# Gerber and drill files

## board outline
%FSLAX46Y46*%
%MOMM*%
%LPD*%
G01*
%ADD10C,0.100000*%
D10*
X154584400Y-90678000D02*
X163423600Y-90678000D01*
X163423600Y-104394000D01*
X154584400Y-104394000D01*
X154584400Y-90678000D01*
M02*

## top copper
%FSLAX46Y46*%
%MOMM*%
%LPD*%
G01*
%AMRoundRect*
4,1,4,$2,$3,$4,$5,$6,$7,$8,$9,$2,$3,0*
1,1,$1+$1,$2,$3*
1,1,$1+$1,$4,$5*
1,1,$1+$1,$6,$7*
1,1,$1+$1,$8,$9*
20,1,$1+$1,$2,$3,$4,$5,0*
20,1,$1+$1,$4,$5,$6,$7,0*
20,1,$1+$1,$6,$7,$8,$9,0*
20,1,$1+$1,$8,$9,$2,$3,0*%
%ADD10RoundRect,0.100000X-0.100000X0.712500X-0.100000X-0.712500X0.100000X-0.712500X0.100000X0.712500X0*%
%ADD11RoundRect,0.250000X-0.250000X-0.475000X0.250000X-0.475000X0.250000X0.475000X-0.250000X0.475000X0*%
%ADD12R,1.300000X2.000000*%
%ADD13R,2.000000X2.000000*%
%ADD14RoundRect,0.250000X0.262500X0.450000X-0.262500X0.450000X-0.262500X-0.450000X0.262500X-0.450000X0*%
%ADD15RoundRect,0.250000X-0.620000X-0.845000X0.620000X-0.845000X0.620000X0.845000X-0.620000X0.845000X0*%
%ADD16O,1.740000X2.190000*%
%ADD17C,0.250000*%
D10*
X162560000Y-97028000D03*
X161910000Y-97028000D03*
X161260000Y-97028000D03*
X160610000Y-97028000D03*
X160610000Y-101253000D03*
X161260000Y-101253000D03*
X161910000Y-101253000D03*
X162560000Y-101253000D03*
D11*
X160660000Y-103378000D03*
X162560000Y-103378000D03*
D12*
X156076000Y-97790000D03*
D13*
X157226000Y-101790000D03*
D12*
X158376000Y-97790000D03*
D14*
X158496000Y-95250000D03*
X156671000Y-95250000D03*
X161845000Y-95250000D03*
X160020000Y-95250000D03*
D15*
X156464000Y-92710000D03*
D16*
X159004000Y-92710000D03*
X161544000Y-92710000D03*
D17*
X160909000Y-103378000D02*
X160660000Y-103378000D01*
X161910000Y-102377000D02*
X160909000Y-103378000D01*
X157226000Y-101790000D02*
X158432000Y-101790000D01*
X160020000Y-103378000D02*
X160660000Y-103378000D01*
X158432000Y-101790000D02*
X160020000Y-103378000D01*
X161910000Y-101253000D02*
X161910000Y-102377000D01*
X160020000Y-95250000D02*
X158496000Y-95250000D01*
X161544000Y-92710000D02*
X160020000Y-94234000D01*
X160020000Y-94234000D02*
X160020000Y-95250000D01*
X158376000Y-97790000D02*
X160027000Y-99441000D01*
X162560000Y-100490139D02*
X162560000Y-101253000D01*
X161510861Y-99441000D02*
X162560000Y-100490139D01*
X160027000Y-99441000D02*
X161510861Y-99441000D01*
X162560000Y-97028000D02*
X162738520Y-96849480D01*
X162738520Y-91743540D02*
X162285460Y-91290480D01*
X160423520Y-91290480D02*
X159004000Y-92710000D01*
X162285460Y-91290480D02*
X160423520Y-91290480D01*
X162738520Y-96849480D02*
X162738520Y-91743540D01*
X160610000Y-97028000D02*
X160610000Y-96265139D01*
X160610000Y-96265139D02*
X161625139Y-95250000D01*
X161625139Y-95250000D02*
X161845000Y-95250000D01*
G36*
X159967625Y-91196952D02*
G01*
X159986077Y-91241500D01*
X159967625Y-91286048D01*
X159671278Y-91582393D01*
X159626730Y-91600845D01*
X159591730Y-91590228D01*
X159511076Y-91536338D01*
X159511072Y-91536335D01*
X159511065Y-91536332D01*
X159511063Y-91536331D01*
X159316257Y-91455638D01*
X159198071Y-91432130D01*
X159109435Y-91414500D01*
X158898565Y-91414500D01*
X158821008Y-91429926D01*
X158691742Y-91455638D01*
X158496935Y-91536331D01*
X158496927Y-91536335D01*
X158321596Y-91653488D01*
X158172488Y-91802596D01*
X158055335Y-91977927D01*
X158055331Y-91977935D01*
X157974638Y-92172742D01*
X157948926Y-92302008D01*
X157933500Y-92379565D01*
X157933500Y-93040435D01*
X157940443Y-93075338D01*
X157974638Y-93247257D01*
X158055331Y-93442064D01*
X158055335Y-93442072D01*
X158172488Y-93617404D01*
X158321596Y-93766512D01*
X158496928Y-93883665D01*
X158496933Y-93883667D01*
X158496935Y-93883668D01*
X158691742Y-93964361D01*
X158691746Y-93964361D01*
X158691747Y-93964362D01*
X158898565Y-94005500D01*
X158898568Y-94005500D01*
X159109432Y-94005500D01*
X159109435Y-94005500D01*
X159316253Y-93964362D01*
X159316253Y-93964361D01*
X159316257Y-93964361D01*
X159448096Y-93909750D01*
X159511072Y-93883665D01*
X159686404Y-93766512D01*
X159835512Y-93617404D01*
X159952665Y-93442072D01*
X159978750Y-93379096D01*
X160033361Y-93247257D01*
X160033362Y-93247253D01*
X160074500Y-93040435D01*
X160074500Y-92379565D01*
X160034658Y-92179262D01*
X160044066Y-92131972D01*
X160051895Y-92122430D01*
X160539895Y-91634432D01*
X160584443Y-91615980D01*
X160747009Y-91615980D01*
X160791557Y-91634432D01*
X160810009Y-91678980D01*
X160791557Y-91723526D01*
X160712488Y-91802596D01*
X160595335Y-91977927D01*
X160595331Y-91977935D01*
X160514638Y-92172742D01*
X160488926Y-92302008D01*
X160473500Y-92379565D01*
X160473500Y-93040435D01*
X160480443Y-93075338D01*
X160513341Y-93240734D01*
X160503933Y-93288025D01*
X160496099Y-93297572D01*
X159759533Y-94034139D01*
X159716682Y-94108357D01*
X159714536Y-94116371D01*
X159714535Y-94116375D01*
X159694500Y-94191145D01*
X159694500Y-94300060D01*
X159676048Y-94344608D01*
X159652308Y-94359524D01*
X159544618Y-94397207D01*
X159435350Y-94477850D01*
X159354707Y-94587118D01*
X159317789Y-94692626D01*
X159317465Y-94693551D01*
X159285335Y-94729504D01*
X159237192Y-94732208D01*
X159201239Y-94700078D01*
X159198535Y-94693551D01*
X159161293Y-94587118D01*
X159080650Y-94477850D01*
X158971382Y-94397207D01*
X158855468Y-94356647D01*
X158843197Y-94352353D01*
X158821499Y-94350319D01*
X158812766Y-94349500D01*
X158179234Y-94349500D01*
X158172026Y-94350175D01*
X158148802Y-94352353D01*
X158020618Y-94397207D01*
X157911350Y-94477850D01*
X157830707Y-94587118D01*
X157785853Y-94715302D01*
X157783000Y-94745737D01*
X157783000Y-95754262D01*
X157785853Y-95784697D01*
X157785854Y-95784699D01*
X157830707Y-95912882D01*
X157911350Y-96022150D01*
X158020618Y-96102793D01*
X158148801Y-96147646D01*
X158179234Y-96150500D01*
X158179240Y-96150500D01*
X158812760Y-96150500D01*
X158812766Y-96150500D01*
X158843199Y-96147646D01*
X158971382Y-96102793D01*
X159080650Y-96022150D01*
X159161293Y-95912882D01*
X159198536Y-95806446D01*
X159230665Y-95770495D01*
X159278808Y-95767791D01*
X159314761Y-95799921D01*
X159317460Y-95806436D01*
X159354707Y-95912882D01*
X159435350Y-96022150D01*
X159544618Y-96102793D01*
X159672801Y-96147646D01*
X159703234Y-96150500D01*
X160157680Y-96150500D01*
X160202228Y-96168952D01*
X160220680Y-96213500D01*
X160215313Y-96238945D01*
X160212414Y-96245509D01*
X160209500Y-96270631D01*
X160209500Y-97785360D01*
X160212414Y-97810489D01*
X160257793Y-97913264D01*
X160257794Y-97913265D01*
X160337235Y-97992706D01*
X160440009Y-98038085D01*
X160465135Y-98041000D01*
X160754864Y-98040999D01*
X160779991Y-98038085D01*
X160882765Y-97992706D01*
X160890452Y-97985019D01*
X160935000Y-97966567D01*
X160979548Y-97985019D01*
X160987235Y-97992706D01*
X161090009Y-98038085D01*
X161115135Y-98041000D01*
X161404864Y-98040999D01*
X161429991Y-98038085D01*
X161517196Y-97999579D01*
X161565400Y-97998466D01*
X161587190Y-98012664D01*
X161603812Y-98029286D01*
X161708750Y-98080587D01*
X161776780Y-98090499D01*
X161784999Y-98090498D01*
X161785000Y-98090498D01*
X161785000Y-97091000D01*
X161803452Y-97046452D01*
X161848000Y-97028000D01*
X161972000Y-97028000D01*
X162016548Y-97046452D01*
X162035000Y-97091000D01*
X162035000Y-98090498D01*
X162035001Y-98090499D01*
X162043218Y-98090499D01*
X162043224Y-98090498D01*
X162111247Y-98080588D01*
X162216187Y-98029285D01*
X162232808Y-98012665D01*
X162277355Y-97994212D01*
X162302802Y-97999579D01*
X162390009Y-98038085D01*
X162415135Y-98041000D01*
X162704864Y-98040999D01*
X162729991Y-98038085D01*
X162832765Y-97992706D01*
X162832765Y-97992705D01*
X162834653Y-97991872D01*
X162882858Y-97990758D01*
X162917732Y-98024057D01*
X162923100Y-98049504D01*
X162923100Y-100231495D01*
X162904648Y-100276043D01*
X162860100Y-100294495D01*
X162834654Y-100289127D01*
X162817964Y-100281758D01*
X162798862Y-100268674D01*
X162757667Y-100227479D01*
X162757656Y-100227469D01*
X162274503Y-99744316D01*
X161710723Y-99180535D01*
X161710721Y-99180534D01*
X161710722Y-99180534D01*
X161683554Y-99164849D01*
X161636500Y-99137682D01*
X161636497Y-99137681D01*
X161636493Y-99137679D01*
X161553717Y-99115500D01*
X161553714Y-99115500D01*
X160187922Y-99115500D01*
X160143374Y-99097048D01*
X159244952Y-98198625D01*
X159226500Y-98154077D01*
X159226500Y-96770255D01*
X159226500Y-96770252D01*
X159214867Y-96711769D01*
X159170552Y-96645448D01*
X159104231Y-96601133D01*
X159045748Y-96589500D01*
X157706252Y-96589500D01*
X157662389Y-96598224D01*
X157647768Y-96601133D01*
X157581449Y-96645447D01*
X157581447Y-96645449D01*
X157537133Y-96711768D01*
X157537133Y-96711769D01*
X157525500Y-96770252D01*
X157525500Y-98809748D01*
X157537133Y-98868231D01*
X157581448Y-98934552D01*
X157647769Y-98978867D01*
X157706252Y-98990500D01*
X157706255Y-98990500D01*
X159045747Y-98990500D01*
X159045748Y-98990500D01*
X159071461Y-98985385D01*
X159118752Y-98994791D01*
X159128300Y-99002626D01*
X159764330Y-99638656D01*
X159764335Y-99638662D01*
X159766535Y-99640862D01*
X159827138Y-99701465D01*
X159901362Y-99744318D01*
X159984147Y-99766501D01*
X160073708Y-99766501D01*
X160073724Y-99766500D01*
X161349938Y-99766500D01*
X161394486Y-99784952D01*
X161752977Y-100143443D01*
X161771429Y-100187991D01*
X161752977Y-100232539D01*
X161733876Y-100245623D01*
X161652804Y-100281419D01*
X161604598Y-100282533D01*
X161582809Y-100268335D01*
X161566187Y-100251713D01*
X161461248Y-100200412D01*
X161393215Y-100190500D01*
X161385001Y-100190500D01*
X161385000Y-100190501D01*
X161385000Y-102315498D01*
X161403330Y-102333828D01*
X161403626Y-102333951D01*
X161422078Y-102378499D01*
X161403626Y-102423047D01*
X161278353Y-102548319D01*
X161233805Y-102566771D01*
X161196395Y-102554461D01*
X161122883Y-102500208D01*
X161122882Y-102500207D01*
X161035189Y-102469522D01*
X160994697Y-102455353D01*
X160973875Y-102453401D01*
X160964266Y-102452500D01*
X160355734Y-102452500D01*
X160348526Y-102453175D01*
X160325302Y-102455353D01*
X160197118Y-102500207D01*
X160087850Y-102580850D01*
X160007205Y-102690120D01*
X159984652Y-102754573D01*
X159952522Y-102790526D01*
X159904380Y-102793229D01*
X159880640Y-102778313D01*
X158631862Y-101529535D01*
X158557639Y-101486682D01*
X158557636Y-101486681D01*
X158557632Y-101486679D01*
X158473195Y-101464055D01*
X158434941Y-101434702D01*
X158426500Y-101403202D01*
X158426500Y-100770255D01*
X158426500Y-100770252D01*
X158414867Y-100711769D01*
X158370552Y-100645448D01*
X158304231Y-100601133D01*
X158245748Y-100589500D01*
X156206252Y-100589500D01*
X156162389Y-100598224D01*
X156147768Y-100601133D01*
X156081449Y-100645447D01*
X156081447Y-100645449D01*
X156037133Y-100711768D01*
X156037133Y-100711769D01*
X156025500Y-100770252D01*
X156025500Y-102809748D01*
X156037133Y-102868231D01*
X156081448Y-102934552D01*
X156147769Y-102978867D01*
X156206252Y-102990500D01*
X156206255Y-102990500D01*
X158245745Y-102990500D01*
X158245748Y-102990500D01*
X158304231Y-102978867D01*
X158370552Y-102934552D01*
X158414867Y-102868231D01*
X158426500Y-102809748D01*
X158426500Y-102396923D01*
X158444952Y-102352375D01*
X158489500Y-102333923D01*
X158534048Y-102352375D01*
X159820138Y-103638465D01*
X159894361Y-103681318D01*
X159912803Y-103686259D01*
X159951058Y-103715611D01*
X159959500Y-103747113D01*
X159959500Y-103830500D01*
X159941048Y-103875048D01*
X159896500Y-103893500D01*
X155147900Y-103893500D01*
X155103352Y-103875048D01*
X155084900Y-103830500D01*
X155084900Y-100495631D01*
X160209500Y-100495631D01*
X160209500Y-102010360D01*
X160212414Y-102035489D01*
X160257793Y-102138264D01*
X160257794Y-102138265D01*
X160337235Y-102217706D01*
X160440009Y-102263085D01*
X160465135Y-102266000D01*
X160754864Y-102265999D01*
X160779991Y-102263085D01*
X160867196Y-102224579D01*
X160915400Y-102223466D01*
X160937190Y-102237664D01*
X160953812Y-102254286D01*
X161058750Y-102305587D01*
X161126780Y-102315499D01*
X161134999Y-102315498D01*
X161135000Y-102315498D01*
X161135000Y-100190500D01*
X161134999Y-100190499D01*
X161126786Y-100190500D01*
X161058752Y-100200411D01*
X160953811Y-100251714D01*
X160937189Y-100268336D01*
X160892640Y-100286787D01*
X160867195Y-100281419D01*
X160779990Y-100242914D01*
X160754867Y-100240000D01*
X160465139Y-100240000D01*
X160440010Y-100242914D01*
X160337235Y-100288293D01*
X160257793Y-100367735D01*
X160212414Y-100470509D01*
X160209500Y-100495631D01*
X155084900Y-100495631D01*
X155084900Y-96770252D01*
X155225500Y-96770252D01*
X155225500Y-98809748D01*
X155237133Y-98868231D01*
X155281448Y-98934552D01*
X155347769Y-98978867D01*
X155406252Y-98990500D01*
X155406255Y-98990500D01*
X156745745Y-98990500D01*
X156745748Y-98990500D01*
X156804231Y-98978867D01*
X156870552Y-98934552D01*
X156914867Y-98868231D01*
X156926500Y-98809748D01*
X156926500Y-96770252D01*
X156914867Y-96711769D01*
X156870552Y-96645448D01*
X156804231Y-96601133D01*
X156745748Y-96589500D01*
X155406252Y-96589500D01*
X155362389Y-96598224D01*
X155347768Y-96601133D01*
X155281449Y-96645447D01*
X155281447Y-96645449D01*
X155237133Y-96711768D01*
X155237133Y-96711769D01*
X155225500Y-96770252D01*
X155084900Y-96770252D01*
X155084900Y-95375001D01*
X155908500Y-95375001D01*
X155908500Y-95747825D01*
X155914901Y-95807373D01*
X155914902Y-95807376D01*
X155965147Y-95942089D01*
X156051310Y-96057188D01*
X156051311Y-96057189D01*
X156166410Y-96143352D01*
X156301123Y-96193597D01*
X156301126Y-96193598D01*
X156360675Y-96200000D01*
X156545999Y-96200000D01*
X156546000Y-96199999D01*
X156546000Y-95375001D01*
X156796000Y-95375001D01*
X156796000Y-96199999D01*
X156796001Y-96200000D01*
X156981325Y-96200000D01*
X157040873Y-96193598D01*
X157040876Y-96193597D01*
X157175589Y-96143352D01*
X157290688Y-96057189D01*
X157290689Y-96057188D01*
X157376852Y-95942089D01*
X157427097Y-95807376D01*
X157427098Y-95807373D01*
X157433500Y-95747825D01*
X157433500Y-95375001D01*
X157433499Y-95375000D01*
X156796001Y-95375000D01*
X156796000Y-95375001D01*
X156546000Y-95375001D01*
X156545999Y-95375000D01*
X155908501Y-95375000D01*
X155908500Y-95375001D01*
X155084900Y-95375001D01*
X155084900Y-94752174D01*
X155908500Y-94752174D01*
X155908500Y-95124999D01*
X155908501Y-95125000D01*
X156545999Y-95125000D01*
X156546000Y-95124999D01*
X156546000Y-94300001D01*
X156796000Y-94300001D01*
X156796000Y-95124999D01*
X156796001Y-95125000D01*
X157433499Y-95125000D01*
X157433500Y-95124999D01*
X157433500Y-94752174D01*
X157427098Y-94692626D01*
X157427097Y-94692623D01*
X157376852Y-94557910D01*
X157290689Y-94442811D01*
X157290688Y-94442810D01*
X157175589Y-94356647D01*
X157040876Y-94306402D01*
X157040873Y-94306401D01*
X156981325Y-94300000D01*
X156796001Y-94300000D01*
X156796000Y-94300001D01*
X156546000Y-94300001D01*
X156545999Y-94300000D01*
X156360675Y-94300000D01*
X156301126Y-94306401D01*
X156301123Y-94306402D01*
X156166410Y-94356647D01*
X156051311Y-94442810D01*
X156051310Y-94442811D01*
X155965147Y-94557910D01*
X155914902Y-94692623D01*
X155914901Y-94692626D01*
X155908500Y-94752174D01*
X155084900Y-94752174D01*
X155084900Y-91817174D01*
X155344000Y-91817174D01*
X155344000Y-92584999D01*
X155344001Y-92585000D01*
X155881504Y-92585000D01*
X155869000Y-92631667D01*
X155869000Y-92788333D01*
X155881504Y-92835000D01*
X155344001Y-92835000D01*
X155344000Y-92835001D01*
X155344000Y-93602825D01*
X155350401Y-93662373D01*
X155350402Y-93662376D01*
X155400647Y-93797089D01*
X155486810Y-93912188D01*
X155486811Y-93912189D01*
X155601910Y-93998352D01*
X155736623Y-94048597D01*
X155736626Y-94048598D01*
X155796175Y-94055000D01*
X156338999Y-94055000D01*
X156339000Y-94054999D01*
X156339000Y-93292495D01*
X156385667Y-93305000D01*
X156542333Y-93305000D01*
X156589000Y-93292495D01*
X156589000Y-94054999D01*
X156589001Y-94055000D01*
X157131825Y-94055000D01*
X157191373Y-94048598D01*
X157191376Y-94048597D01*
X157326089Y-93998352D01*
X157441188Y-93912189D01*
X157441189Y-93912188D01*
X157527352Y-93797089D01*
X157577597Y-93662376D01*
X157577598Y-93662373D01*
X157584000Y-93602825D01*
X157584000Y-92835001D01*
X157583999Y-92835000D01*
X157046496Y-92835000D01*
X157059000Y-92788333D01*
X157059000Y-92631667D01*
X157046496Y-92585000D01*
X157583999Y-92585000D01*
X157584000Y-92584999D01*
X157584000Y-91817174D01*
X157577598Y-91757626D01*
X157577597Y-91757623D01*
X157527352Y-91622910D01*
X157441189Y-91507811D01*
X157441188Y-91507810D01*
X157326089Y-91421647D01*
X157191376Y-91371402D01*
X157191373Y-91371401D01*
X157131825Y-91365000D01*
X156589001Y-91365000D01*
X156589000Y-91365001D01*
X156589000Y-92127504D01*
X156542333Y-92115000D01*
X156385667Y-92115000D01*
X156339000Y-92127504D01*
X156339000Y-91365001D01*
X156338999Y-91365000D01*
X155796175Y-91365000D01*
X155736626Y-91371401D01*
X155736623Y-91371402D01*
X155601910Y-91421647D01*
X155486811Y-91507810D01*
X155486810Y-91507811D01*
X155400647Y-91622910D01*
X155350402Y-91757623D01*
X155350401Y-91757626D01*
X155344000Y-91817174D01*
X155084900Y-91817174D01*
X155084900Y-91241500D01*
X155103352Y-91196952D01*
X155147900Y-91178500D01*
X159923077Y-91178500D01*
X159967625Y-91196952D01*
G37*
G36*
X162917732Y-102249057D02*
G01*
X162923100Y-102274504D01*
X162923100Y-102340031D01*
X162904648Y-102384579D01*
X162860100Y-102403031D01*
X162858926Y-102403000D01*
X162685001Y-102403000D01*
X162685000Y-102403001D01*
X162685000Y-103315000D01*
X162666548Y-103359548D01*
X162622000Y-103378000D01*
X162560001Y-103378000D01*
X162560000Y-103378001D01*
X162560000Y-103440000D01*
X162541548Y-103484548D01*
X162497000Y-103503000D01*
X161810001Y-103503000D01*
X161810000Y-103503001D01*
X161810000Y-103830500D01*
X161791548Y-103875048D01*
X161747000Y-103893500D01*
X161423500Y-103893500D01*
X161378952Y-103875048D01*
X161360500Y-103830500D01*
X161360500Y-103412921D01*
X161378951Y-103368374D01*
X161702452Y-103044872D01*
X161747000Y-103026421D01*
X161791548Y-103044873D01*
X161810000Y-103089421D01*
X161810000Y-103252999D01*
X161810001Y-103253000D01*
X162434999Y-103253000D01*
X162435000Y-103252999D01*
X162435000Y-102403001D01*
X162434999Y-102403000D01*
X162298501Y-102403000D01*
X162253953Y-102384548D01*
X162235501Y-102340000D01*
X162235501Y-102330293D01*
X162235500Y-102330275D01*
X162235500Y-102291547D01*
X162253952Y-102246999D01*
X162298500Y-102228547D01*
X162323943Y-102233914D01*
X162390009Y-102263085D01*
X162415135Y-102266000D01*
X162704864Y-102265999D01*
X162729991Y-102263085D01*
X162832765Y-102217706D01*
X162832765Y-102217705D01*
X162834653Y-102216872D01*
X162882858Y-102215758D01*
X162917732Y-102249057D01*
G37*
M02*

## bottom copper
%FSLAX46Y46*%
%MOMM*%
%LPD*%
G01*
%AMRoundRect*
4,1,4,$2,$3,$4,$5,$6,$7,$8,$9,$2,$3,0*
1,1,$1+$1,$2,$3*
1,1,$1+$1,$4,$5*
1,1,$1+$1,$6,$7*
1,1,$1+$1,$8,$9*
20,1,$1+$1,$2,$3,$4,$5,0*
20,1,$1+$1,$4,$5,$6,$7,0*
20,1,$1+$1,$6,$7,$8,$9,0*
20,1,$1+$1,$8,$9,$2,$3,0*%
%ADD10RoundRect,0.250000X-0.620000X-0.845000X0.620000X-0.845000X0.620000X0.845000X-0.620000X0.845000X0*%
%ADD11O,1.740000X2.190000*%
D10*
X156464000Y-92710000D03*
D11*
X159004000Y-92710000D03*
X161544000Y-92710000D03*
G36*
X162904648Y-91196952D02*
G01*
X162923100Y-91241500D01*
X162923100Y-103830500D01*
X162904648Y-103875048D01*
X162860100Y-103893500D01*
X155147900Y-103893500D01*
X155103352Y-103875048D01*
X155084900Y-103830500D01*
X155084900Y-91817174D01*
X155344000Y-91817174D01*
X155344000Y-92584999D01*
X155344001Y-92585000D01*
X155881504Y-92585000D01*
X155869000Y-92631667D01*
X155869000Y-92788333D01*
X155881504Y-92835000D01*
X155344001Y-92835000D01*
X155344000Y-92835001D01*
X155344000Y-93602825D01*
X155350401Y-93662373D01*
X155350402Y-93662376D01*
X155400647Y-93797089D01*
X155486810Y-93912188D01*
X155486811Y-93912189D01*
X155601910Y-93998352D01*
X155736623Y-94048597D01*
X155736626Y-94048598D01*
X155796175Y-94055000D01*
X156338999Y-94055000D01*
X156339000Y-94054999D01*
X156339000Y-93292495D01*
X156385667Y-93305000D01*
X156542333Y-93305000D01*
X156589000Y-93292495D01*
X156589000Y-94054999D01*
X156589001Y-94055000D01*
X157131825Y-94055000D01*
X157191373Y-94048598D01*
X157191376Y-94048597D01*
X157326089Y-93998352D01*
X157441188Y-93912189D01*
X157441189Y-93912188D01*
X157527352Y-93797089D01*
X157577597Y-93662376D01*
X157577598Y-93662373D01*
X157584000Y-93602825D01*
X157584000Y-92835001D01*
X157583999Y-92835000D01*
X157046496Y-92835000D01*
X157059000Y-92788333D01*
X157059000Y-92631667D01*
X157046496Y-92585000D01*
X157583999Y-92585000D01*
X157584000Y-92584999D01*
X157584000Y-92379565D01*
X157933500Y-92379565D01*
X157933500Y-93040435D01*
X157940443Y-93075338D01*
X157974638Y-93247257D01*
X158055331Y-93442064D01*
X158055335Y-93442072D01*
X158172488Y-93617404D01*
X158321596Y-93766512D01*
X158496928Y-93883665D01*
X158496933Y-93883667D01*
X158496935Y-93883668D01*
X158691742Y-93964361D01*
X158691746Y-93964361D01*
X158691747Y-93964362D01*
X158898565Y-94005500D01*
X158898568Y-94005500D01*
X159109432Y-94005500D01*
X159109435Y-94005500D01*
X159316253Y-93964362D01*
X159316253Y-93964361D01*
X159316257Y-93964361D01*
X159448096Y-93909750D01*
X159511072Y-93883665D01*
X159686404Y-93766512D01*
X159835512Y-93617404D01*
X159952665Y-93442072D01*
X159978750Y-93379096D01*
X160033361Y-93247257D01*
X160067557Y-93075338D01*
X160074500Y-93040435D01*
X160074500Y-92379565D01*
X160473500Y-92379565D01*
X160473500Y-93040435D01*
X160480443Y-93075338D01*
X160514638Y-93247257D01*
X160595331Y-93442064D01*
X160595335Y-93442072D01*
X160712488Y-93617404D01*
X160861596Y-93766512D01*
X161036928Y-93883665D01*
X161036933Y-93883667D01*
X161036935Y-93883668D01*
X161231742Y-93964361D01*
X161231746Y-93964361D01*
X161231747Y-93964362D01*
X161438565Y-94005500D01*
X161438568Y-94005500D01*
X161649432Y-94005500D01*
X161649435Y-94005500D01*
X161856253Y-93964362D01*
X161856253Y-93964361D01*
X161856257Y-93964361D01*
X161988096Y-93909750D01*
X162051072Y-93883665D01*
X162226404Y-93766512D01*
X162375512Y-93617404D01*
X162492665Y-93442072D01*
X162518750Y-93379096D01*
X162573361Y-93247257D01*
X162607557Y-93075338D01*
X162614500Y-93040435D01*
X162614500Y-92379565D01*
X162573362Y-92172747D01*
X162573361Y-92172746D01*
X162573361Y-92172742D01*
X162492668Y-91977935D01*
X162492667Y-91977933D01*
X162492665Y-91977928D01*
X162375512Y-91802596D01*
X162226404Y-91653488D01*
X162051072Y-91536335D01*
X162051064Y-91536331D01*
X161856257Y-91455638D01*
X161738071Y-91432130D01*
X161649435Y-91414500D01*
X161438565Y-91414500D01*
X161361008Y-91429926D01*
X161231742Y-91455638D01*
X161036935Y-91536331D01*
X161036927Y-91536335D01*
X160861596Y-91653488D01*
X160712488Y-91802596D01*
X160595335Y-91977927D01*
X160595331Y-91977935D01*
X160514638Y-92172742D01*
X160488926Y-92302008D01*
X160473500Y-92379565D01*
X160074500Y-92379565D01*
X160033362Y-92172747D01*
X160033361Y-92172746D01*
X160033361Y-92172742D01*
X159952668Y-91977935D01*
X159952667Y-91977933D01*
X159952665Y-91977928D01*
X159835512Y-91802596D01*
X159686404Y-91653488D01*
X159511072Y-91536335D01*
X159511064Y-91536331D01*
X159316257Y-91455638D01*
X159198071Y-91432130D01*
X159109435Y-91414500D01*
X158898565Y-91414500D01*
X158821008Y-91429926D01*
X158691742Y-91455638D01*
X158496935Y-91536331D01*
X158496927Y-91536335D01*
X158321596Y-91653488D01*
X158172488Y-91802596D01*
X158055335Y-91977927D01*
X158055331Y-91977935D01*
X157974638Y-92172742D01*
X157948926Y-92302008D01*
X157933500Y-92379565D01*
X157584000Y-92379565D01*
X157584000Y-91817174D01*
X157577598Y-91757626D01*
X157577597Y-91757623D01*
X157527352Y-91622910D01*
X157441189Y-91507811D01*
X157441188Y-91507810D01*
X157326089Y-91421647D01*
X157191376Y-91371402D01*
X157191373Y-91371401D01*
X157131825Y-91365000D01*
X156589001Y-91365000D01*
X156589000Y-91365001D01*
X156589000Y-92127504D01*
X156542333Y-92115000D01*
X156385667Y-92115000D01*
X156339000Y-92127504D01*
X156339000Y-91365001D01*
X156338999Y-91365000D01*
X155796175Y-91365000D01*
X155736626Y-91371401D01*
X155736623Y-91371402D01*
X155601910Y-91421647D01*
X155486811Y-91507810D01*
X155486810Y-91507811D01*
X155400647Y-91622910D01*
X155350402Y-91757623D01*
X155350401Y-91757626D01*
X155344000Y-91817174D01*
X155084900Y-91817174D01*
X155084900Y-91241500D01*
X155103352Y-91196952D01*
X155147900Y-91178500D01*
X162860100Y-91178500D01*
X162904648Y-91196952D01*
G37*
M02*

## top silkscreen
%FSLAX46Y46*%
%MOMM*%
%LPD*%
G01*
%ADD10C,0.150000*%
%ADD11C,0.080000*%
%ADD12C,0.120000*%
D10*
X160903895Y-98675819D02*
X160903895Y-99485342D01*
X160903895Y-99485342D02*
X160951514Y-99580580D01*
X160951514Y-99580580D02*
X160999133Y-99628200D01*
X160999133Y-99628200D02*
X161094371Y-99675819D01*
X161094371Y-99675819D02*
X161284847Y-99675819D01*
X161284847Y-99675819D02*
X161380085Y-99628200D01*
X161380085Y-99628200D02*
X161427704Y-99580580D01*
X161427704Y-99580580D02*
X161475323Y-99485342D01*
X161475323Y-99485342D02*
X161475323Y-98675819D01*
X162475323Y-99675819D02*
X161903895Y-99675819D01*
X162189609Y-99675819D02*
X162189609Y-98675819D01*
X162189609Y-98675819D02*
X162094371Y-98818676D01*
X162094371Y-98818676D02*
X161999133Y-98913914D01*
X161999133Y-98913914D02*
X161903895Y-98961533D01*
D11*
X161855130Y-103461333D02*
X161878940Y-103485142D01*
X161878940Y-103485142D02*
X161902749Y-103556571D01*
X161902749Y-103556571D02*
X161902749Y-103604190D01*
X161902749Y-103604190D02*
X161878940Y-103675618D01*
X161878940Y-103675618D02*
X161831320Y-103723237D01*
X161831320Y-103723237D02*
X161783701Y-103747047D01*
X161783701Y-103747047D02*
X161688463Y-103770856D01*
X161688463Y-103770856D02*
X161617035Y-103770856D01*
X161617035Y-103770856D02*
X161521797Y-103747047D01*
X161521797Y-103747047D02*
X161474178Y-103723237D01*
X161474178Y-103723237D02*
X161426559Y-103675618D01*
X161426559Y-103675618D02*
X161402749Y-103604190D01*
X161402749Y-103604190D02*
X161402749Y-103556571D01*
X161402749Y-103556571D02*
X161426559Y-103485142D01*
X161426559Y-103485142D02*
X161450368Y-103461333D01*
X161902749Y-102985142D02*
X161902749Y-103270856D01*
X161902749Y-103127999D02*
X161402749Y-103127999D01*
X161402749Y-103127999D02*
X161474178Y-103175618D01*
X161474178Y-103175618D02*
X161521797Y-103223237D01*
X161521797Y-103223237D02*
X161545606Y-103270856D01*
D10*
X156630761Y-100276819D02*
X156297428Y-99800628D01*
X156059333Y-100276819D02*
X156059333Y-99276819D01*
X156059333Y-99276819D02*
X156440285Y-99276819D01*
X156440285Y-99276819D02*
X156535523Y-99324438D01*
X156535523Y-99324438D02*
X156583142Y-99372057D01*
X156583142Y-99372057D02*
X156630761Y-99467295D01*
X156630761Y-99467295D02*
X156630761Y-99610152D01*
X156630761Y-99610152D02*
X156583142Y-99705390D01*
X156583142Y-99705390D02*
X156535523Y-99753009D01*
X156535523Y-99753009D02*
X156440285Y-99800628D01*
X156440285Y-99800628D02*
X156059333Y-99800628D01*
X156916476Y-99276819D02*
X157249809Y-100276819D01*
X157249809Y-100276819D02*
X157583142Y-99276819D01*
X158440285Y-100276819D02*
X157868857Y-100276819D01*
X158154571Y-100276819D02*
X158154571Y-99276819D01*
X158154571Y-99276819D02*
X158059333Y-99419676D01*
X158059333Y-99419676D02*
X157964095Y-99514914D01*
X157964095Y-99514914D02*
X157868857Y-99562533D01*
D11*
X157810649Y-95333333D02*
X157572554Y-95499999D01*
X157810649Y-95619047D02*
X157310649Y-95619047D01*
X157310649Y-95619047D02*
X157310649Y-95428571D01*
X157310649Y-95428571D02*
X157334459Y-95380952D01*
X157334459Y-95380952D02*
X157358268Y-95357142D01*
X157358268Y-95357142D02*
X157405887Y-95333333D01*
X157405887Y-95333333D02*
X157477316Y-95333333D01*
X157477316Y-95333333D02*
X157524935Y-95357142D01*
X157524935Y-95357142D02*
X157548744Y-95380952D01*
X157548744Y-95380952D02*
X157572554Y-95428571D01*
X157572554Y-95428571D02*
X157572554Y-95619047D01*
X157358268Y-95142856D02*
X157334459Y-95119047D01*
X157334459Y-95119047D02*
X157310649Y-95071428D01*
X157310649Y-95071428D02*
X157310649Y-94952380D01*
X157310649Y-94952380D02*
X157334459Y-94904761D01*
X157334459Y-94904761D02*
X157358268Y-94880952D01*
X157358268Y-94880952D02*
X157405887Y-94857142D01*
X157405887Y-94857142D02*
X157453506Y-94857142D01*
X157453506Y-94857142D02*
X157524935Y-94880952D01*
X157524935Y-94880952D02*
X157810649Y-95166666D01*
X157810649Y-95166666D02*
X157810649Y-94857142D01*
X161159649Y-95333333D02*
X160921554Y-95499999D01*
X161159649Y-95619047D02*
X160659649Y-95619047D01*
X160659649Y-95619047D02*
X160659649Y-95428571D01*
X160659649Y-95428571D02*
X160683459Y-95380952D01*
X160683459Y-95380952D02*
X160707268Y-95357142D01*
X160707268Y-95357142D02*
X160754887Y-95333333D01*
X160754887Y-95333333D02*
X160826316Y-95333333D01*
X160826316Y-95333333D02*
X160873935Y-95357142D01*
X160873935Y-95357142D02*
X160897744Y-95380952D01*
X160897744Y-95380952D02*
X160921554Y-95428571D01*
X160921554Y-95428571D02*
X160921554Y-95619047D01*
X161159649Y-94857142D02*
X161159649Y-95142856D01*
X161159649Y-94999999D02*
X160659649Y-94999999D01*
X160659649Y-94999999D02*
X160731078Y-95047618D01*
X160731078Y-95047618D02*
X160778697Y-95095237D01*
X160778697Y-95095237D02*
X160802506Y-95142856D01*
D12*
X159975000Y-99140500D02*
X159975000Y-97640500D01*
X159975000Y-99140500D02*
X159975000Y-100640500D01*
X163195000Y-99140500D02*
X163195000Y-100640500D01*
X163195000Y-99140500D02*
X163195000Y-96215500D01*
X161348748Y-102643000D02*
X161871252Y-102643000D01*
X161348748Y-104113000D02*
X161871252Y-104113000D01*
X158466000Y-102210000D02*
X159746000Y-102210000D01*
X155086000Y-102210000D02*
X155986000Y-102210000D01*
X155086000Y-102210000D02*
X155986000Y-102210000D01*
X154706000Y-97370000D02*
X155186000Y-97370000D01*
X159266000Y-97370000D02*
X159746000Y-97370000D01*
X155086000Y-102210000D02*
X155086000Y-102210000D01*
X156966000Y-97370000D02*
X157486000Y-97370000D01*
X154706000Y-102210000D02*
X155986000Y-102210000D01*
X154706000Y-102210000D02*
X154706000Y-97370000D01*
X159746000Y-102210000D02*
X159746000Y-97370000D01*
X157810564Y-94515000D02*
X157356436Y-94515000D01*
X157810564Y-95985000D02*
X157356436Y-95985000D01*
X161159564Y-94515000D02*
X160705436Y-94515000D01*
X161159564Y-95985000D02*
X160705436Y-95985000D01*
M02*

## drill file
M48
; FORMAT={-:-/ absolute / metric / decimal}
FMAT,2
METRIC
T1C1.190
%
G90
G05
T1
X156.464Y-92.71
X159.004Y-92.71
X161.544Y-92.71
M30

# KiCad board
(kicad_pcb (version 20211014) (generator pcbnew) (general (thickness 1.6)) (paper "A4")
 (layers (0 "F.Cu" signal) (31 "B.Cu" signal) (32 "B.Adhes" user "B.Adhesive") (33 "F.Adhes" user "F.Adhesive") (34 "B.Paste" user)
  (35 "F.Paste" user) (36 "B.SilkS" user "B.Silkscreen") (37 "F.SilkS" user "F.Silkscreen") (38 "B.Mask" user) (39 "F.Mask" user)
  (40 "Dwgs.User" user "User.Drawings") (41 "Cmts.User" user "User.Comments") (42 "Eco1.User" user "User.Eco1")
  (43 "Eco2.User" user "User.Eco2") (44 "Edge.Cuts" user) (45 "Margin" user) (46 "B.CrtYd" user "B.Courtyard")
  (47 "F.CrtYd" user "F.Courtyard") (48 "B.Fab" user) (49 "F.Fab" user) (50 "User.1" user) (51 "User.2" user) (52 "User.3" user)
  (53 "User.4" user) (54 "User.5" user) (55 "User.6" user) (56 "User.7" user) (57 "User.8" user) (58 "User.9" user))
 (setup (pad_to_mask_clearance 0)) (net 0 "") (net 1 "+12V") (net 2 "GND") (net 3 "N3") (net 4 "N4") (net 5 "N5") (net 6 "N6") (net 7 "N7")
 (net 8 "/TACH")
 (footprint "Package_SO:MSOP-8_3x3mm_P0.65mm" (layer "F.Cu") (at 161.585 99.1405 -90)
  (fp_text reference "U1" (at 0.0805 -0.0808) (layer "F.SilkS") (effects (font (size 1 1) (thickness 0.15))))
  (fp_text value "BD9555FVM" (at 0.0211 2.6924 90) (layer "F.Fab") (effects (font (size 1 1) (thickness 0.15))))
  (fp_line (start 0 1.61) (end -1.5 1.61) (layer "F.SilkS") (width 0.12))
  (fp_line (start 0 1.61) (end 1.5 1.61) (layer "F.SilkS") (width 0.12))
  (fp_line (start 0 -1.61) (end 1.5 -1.61) (layer "F.SilkS") (width 0.12))
  (fp_line (start 0 -1.61) (end -2.925 -1.61) (layer "F.SilkS") (width 0.12))
  (pad "1" smd roundrect (at -2.1125 -0.975 270) (size 1.625 0.4) (layers "F.Cu" "F.Paste" "F.Mask") (roundrect_rratio 0.25) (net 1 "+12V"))
  (pad "2" smd roundrect (at -2.1125 -0.325 270) (size 1.625 0.4) (layers "F.Cu" "F.Paste" "F.Mask") (roundrect_rratio 0.25) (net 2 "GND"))
  (pad "3" smd roundrect (at -2.1125 0.325 270) (size 1.625 0.4) (layers "F.Cu" "F.Paste" "F.Mask") (roundrect_rratio 0.25) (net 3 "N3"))
  (pad "4" smd roundrect (at -2.1125 0.975 270) (size 1.625 0.4) (layers "F.Cu" "F.Paste" "F.Mask") (roundrect_rratio 0.25) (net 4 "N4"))
  (pad "5" smd roundrect (at 2.1125 0.975 270) (size 1.625 0.4) (layers "F.Cu" "F.Paste" "F.Mask") (roundrect_rratio 0.25))
  (pad "6" smd roundrect (at 2.1125 0.325 270) (size 1.625 0.4) (layers "F.Cu" "F.Paste" "F.Mask") (roundrect_rratio 0.25) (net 2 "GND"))
  (pad "7" smd roundrect (at 2.1125 -0.325 270) (size 1.625 0.4) (layers "F.Cu" "F.Paste" "F.Mask") (roundrect_rratio 0.25) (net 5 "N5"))
  (pad "8" smd roundrect (at 2.1125 -0.975 270) (size 1.625 0.4) (layers "F.Cu" "F.Paste" "F.Mask") (roundrect_rratio 0.25) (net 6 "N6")))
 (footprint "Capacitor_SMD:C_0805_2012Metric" (layer "F.Cu") (at 161.61 103.378)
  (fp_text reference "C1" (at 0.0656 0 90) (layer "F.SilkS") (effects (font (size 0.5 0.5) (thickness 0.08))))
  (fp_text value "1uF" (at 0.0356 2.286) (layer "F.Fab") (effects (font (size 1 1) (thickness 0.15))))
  (fp_line (start -0.261252 -0.735) (end 0.261252 -0.735) (layer "F.SilkS") (width 0.12))
  (fp_line (start -0.261252 0.735) (end 0.261252 0.735) (layer "F.SilkS") (width 0.12))
  (pad "1" smd roundrect (at -0.95 0) (size 1 1.45) (layers "F.Cu" "F.Paste" "F.Mask") (roundrect_rratio 0.25) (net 5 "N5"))
  (pad "2" smd roundrect (at 0.95 0) (size 1 1.45) (layers "F.Cu" "F.Paste" "F.Mask") (roundrect_rratio 0.25) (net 2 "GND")))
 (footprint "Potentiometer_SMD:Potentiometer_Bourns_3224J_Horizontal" (layer "F.Cu") (at 157.226 99.79 90)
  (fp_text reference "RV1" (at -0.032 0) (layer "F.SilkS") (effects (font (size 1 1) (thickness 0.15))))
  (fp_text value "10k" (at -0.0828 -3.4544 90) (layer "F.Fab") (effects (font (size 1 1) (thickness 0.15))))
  (fp_line (start -2.42 1.24) (end -2.42 2.52) (layer "F.SilkS") (width 0.12))
  (fp_line (start -2.42 -2.14) (end -2.42 -1.24) (layer "F.SilkS") (width 0.12))
  (fp_line (start -2.42 -2.14) (end -2.42 -1.24) (layer "F.SilkS") (width 0.12))
  (fp_line (start 2.42 -2.52) (end 2.42 -2.04) (layer "F.SilkS") (width 0.12))
  (fp_line (start 2.42 2.04) (end 2.42 2.52) (layer "F.SilkS") (width 0.12))
  (fp_line (start -2.42 -2.14) (end -2.42 -2.14) (layer "F.SilkS") (width 0.12))
  (fp_line (start 2.42 -0.26) (end 2.42 0.26) (layer "F.SilkS") (width 0.12))
  (fp_line (start -2.42 -2.52) (end -2.42 -1.24) (layer "F.SilkS") (width 0.12))
  (fp_line (start -2.42 -2.52) (end 2.42 -2.52) (layer "F.SilkS") (width 0.12))
  (fp_line (start -2.42 2.52) (end 2.42 2.52) (layer "F.SilkS") (width 0.12))
  (pad "1" smd rect (at 2 -1.15 90) (size 2 1.3) (layers "F.Cu" "F.Paste" "F.Mask") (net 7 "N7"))
  (pad "2" smd rect (at -2 0 90) (size 2 2) (layers "F.Cu" "F.Paste" "F.Mask") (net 5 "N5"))
  (pad "3" smd rect (at 2 1.15 90) (size 2 1.3) (layers "F.Cu" "F.Paste" "F.Mask") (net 6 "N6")))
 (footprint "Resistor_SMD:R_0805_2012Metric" (layer "F.Cu") (at 157.5835 95.25 180)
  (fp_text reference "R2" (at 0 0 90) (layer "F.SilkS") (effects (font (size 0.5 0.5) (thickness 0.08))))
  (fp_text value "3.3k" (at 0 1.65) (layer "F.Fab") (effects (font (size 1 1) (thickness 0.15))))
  (fp_line (start -0.227064 0.735) (end 0.227064 0.735) (layer "F.SilkS") (width 0.12))
  (fp_line (start -0.227064 -0.735) (end 0.227064 -0.735) (layer "F.SilkS") (width 0.12))
  (pad "1" smd roundrect (at -0.9125 0 180) (size 1.025 1.4) (layers "F.Cu" "F.Paste" "F.Mask") (roundrect_rratio 0.243902) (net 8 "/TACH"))
  (pad "2" smd roundrect (at 0.9125 0 180) (size 1.025 1.4) (layers "F.Cu" "F.Paste" "F.Mask") (roundrect_rratio 0.243902) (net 2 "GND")))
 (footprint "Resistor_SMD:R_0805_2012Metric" (layer "F.Cu") (at 160.9325 95.25 180)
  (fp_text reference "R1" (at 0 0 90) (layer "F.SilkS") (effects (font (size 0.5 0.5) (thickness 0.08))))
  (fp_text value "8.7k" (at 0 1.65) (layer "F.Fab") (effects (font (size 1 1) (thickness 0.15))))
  (fp_line (start -0.227064 0.735) (end 0.227064 0.735) (layer "F.SilkS") (width 0.12))
  (fp_line (start -0.227064 -0.735) (end 0.227064 -0.735) (layer "F.SilkS") (width 0.12))
  (pad "1" smd roundrect (at -0.9125 0 180) (size 1.025 1.4) (layers "F.Cu" "F.Paste" "F.Mask") (roundrect_rratio 0.243902) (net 4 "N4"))
  (pad "2" smd roundrect (at 0.9125 0 180) (size 1.025 1.4) (layers "F.Cu" "F.Paste" "F.Mask") (roundrect_rratio 0.243902) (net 8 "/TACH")))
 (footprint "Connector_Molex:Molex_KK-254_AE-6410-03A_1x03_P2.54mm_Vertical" (layer "B.Cu") (at 156.464 92.71)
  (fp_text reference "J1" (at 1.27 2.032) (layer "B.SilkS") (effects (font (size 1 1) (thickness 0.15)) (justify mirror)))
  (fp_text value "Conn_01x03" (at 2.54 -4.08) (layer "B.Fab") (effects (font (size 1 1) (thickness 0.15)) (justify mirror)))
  (pad "1" thru_hole roundrect (at 0 0) (size 1.74 2.19) (drill 1.19) (layers *.Cu *.Mask) (roundrect_rratio 0.143678) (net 2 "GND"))
  (pad "2" thru_hole oval (at 2.54 0) (size 1.74 2.19) (drill 1.19) (layers *.Cu *.Mask) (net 1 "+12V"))
  (pad "3" thru_hole oval (at 5.08 0) (size 1.74 2.19) (drill 1.19) (layers *.Cu *.Mask) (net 8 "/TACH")))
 (gr_rect (start 163.4236 90.678) (end 154.5844 104.394) (layer "Edge.Cuts") (width 0.1) (fill none))
 (segment (start 160.909 103.378) (end 160.66 103.378) (width 0.25) (layer "F.Cu") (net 5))
 (segment (start 161.91 102.377) (end 160.909 103.378) (width 0.25) (layer "F.Cu") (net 5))
 (segment (start 157.226 101.79) (end 158.432 101.79) (width 0.25) (layer "F.Cu") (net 5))
 (segment (start 160.02 103.378) (end 160.66 103.378) (width 0.25) (layer "F.Cu") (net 5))
 (segment (start 158.432 101.79) (end 160.02 103.378) (width 0.25) (layer "F.Cu") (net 5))
 (segment (start 161.91 101.253) (end 161.91 102.377) (width 0.25) (layer "F.Cu") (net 5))
 (segment (start 160.02 95.25) (end 158.496 95.25) (width 0.25) (layer "F.Cu") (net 8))
 (segment (start 161.544 92.71) (end 160.02 94.234) (width 0.25) (layer "F.Cu") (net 8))
 (segment (start 160.02 94.234) (end 160.02 95.25) (width 0.25) (layer "F.Cu") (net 8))
 (segment (start 158.376 97.79) (end 160.027 99.441) (width 0.25) (layer "F.Cu") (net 6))
 (segment (start 162.56 100.490139) (end 162.56 101.253) (width 0.25) (layer "F.Cu") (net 6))
 (segment (start 161.510861 99.441) (end 162.56 100.490139) (width 0.25) (layer "F.Cu") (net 6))
 (segment (start 160.027 99.441) (end 161.510861 99.441) (width 0.25) (layer "F.Cu") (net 6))
 (segment (start 162.56 97.028) (end 162.73852 96.84948) (width 0.25) (layer "F.Cu") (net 1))
 (segment (start 162.73852 91.74354) (end 162.28546 91.29048) (width 0.25) (layer "F.Cu") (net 1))
 (segment (start 160.42352 91.29048) (end 159.004 92.71) (width 0.25) (layer "F.Cu") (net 1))
 (segment (start 162.28546 91.29048) (end 160.42352 91.29048) (width 0.25) (layer "F.Cu") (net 1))
 (segment (start 162.73852 96.84948) (end 162.73852 91.74354) (width 0.25) (layer "F.Cu") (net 1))
 (segment (start 160.61 97.028) (end 160.61 96.265139) (width 0.25) (layer "F.Cu") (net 4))
 (segment (start 160.61 96.265139) (end 161.625139 95.25) (width 0.25) (layer "F.Cu") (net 4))
 (segment (start 161.625139 95.25) (end 161.845 95.25) (width 0.25) (layer "F.Cu") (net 4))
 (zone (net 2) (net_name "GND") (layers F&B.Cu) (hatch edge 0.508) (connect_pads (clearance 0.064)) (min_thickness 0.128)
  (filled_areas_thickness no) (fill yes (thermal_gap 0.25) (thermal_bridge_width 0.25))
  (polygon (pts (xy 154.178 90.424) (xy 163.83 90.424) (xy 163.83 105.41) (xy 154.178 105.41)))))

